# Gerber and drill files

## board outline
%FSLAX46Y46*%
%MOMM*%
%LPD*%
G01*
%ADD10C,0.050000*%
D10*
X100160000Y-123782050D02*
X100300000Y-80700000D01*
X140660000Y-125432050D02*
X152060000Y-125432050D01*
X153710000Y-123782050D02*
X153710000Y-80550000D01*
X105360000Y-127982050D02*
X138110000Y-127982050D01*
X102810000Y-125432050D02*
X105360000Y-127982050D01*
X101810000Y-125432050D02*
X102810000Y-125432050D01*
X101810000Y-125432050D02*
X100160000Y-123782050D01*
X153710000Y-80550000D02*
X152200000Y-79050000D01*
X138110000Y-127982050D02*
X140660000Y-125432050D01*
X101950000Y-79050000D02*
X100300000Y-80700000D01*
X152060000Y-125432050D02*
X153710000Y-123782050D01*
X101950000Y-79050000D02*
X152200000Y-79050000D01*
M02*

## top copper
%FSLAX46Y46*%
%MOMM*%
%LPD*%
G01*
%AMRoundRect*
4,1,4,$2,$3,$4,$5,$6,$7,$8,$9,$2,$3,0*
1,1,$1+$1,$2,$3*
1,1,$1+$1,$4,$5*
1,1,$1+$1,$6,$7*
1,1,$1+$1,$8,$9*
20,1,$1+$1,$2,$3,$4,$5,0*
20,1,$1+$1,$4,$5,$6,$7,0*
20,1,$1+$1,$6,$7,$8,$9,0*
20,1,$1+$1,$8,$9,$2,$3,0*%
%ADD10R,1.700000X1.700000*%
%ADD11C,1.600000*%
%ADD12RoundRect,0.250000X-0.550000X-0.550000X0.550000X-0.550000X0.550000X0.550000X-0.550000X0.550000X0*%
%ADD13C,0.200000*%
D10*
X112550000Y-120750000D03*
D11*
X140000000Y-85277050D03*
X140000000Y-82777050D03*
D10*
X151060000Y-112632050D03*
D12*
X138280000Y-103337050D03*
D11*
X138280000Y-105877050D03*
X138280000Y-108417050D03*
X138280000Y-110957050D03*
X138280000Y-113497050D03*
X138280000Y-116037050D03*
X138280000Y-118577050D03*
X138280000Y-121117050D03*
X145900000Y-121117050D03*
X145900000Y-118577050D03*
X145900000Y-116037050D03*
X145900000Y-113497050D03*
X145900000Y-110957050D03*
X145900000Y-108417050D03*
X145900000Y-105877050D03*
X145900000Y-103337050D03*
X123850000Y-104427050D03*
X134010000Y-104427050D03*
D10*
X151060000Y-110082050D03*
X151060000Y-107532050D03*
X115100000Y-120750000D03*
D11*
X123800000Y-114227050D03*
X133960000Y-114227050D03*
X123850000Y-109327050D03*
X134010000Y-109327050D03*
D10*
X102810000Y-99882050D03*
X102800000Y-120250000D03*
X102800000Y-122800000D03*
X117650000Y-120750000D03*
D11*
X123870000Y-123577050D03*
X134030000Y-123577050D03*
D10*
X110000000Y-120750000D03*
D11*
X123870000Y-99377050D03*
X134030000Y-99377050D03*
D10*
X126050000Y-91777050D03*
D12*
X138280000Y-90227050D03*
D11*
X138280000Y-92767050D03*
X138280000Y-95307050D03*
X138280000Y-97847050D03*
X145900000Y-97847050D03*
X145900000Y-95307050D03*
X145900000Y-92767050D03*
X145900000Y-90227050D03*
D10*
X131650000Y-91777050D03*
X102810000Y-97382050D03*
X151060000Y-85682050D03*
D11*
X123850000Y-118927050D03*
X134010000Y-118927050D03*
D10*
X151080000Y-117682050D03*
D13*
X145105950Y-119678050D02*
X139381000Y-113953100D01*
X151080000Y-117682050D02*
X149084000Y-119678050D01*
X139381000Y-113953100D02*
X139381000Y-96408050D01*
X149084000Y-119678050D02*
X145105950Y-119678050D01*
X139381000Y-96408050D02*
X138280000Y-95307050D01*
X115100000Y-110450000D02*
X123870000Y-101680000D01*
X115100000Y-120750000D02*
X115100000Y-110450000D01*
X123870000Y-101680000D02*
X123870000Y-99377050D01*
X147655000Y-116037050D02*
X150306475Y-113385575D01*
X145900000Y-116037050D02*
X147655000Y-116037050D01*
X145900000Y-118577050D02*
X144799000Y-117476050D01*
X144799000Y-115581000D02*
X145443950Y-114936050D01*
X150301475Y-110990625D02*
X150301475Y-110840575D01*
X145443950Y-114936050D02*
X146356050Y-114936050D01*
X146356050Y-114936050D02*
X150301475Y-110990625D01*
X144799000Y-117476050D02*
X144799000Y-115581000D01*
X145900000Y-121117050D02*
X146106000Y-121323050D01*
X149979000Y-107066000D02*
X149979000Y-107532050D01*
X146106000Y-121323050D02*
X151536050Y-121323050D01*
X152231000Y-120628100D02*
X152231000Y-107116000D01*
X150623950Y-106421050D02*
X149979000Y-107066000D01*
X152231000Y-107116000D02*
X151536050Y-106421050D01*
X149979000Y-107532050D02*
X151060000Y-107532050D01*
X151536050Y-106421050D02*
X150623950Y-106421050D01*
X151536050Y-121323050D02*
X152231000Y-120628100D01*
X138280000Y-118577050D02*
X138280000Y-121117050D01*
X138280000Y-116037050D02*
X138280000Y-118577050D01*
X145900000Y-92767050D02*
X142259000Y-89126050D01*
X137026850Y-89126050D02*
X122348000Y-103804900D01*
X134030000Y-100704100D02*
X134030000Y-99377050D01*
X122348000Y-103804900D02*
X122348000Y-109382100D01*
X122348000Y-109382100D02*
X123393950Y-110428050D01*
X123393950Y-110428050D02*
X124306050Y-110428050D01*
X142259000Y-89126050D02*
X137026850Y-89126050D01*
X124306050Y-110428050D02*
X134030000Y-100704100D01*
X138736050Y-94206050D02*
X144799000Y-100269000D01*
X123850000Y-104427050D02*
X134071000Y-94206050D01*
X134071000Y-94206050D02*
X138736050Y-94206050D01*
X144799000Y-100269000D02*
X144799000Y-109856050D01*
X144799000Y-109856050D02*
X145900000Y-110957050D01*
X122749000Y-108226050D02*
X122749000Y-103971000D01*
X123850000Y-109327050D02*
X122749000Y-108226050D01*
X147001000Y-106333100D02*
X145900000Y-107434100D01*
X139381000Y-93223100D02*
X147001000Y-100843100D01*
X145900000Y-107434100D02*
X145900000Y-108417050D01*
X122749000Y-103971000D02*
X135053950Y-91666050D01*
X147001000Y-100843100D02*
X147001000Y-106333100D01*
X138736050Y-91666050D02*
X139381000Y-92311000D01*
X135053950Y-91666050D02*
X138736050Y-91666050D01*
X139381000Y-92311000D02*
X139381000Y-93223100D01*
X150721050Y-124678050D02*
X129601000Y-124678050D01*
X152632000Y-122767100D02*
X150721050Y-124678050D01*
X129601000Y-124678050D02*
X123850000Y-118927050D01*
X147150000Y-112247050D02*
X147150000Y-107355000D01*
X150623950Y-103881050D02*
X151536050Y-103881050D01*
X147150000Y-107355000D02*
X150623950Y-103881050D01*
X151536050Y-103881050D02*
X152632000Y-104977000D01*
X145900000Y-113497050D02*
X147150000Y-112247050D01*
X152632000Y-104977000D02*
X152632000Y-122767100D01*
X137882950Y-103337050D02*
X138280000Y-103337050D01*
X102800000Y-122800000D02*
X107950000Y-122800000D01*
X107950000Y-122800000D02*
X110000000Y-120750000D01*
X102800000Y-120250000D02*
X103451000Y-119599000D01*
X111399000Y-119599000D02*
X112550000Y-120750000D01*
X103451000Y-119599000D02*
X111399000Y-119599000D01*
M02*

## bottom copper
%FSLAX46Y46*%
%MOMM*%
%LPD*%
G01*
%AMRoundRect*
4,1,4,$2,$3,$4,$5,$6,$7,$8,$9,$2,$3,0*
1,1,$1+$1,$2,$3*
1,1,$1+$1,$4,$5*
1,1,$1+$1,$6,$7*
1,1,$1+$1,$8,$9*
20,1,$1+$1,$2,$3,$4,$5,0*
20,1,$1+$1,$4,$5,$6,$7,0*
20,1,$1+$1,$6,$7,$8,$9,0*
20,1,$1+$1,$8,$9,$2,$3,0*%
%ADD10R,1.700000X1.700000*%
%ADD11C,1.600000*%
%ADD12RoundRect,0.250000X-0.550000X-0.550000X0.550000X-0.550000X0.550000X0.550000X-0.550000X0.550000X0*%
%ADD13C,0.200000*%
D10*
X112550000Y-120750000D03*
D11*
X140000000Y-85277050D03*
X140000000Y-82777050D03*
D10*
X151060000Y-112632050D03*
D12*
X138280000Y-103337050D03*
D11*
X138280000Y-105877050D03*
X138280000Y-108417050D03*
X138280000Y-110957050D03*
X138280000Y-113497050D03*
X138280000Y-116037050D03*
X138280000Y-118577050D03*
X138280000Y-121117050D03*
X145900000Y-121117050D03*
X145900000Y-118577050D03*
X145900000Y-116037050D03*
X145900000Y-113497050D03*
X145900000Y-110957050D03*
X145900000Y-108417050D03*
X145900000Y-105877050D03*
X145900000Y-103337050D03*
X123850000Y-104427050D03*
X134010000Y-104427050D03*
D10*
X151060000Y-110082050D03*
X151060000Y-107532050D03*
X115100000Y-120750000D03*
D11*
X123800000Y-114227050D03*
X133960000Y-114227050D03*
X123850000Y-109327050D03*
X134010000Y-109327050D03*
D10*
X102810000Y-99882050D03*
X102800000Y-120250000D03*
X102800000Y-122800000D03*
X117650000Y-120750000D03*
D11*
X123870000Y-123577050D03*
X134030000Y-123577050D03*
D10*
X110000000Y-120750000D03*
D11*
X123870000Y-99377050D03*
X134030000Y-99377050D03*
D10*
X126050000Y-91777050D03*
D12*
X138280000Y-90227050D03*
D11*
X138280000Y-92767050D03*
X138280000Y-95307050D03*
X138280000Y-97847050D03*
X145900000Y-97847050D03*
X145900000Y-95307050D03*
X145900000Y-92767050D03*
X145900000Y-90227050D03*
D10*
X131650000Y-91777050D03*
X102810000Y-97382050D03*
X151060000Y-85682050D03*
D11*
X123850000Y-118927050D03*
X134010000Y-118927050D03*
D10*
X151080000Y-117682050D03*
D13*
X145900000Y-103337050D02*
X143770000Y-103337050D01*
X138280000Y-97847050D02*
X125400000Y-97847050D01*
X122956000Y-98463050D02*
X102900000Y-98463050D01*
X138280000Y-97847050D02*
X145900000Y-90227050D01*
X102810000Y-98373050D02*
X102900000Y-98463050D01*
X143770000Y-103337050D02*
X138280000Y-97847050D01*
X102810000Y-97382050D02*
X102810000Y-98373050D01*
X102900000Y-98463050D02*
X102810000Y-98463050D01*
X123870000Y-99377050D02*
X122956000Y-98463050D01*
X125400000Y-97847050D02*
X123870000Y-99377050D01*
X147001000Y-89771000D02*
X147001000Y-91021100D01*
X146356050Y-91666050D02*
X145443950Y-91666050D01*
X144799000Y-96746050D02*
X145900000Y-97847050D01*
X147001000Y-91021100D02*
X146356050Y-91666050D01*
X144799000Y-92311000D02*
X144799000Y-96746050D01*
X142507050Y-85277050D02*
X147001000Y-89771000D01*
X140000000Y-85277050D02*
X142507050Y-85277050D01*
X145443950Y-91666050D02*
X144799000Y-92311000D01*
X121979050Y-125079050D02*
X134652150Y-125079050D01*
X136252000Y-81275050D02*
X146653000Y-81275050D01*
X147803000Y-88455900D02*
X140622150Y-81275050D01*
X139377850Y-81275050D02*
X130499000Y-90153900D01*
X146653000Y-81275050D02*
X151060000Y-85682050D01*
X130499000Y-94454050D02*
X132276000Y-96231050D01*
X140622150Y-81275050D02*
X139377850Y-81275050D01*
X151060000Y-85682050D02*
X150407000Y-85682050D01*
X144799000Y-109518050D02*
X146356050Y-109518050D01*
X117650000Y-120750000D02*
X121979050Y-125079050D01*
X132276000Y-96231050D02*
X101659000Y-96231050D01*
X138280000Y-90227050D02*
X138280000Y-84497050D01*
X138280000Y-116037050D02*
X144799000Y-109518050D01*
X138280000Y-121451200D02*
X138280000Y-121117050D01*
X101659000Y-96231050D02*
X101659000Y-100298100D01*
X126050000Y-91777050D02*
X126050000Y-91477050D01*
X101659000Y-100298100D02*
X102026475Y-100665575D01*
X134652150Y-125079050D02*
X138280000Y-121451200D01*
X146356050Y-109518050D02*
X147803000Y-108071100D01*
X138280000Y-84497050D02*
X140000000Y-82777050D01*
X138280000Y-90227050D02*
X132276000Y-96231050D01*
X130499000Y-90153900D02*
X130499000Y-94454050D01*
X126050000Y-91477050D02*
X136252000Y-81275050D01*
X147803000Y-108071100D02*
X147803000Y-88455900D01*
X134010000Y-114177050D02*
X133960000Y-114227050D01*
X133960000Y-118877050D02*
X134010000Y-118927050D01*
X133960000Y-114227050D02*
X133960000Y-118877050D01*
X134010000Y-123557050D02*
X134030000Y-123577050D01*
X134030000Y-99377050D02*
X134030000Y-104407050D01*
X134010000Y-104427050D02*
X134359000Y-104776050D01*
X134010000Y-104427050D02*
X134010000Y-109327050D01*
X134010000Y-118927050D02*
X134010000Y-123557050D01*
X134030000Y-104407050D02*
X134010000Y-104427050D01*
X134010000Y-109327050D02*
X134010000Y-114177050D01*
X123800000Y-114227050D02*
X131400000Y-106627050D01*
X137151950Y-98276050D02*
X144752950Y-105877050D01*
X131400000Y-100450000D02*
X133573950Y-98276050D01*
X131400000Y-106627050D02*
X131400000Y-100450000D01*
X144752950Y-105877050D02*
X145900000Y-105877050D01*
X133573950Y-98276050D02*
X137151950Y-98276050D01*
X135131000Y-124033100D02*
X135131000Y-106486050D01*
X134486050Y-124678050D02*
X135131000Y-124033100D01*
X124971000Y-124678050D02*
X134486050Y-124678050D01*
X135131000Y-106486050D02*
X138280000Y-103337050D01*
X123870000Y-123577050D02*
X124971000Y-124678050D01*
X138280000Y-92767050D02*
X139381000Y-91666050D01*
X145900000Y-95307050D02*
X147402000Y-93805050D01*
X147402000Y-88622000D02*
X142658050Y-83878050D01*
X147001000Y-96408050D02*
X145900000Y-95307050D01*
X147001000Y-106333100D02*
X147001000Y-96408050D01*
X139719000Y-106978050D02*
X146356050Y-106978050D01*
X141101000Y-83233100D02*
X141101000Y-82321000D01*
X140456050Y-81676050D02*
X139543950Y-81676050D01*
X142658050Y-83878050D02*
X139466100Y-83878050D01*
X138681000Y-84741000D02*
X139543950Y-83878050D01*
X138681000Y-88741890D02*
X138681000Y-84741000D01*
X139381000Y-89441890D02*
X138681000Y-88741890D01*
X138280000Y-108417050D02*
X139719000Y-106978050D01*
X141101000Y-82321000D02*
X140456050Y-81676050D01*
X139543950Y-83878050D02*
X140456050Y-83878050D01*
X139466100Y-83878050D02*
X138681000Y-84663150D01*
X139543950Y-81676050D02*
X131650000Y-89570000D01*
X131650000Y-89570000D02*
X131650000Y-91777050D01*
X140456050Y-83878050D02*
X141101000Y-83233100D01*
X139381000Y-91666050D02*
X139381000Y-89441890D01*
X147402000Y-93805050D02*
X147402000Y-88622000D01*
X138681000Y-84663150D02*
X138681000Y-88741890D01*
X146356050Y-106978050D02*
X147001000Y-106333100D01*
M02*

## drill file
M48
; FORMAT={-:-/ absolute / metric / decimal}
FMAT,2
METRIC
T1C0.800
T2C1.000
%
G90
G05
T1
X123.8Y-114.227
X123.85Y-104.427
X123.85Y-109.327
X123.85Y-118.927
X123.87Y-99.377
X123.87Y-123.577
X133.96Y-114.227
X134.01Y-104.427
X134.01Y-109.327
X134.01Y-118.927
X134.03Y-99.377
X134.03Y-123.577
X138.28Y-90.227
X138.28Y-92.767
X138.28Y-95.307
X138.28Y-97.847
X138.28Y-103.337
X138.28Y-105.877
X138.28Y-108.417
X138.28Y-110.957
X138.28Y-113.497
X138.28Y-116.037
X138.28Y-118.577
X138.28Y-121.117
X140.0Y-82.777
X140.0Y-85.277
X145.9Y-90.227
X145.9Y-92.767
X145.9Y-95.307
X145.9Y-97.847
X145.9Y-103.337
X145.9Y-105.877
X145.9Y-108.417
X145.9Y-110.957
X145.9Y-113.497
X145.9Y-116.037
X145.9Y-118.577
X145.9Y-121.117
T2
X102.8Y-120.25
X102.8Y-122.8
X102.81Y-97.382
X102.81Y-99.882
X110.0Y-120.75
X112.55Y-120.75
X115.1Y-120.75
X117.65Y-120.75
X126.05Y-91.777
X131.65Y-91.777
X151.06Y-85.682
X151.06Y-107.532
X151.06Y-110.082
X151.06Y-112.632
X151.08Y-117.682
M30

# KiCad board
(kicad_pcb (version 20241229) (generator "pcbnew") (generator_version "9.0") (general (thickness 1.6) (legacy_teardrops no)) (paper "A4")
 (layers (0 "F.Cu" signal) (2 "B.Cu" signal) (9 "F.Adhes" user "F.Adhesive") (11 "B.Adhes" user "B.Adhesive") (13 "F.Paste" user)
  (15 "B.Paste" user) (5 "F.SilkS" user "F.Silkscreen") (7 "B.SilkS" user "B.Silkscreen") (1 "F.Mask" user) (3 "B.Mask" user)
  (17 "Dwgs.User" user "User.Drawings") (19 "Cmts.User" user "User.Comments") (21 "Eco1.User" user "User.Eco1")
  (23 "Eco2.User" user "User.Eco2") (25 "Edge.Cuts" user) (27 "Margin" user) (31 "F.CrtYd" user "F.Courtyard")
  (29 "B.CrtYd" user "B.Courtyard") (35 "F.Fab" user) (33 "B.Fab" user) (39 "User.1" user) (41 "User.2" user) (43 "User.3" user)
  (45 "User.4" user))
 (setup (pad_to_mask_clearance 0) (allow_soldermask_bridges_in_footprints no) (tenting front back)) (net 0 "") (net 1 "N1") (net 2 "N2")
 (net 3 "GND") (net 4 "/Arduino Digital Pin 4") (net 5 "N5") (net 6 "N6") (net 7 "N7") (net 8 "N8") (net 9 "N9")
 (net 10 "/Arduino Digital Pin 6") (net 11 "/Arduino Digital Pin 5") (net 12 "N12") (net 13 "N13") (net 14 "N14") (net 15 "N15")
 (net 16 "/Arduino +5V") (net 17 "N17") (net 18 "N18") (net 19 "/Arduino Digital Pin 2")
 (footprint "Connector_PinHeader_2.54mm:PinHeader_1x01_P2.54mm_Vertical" (layer "F.Cu") (at 112.55 120.75)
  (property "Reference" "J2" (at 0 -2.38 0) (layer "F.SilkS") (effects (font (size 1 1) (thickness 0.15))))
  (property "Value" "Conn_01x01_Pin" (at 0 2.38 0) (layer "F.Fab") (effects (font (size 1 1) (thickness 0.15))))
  (pad "1" thru_hole rect (at 0 0) (size 1.7 1.7) (drill 1) (layers "*.Cu" "*.Mask") (remove_unused_layers no) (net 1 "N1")))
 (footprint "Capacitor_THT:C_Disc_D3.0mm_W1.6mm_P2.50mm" (layer "F.Cu") (at 140 85.27705 90)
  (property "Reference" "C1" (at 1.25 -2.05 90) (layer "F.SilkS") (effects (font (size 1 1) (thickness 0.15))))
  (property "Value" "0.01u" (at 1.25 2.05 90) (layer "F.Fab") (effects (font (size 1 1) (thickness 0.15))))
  (pad "1" thru_hole circle (at 0 0 90) (size 1.6 1.6) (drill 0.8) (layers "*.Cu" "*.Mask") (remove_unused_layers no) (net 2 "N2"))
  (pad "2" thru_hole circle (at 2.5 0 90) (size 1.6 1.6) (drill 0.8) (layers "*.Cu" "*.Mask") (remove_unused_layers no) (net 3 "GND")))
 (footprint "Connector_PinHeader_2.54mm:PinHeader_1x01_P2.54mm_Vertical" (layer "F.Cu") (at 151.06 112.63205)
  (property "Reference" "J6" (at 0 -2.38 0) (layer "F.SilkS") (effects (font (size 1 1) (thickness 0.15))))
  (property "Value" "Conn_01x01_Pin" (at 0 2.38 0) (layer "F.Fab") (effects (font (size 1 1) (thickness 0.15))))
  (pad "1" thru_hole rect (at 0 0) (size 1.7 1.7) (drill 1) (layers "*.Cu" "*.Mask") (remove_unused_layers no)
   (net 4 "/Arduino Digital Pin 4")))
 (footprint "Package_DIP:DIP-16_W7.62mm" (layer "F.Cu") (at 138.28 103.33705)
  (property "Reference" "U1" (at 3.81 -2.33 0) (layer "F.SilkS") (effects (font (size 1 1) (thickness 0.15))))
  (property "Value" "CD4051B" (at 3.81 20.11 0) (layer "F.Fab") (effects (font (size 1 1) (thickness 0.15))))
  (pad "1" thru_hole roundrect (at 0 0) (size 1.6 1.6) (drill 0.8) (layers "*.Cu" "*.Mask") (remove_unused_layers no)
   (roundrect_rratio 0.15625) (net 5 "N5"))
  (pad "2" thru_hole circle (at 0 2.54) (size 1.6 1.6) (drill 0.8) (layers "*.Cu" "*.Mask") (remove_unused_layers no) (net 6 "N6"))
  (pad "3" thru_hole circle (at 0 5.08) (size 1.6 1.6) (drill 0.8) (layers "*.Cu" "*.Mask") (remove_unused_layers no) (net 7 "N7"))
  (pad "4" thru_hole circle (at 0 7.62) (size 1.6 1.6) (drill 0.8) (layers "*.Cu" "*.Mask") (remove_unused_layers no) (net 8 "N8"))
  (pad "5" thru_hole circle (at 0 10.16) (size 1.6 1.6) (drill 0.8) (layers "*.Cu" "*.Mask") (remove_unused_layers no) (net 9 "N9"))
  (pad "6" thru_hole circle (at 0 12.7) (size 1.6 1.6) (drill 0.8) (layers "*.Cu" "*.Mask") (remove_unused_layers no) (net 3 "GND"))
  (pad "7" thru_hole circle (at 0 15.24) (size 1.6 1.6) (drill 0.8) (layers "*.Cu" "*.Mask") (remove_unused_layers no) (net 3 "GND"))
  (pad "8" thru_hole circle (at 0 17.78) (size 1.6 1.6) (drill 0.8) (layers "*.Cu" "*.Mask") (remove_unused_layers no) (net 3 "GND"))
  (pad "9" thru_hole circle (at 7.62 17.78) (size 1.6 1.6) (drill 0.8) (layers "*.Cu" "*.Mask") (remove_unused_layers no)
   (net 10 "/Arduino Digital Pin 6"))
  (pad "10" thru_hole circle (at 7.62 15.24) (size 1.6 1.6) (drill 0.8) (layers "*.Cu" "*.Mask") (remove_unused_layers no)
   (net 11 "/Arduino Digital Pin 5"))
  (pad "11" thru_hole circle (at 7.62 12.7) (size 1.6 1.6) (drill 0.8) (layers "*.Cu" "*.Mask") (remove_unused_layers no)
   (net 4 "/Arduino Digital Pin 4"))
  (pad "12" thru_hole circle (at 7.62 10.16) (size 1.6 1.6) (drill 0.8) (layers "*.Cu" "*.Mask") (remove_unused_layers no) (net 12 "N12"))
  (pad "13" thru_hole circle (at 7.62 7.62) (size 1.6 1.6) (drill 0.8) (layers "*.Cu" "*.Mask") (remove_unused_layers no) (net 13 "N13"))
  (pad "14" thru_hole circle (at 7.62 5.08) (size 1.6 1.6) (drill 0.8) (layers "*.Cu" "*.Mask") (remove_unused_layers no) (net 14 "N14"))
  (pad "15" thru_hole circle (at 7.62 2.54) (size 1.6 1.6) (drill 0.8) (layers "*.Cu" "*.Mask") (remove_unused_layers no) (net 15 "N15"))
  (pad "16" thru_hole circle (at 7.62 0) (size 1.6 1.6) (drill 0.8) (layers "*.Cu" "*.Mask") (remove_unused_layers no)
   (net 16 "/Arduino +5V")))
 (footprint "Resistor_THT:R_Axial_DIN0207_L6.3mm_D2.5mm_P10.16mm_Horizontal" (layer "F.Cu") (at 123.85 104.42705)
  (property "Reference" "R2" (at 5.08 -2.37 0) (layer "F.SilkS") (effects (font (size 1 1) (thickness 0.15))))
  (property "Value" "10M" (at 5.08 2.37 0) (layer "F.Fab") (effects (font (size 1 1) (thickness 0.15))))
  (pad "1" thru_hole circle (at 0 0) (size 1.6 1.6) (drill 0.8) (layers "*.Cu" "*.Mask") (remove_unused_layers no) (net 13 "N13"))
  (pad "2" thru_hole circle (at 10.16 0) (size 1.6 1.6) (drill 0.8) (layers "*.Cu" "*.Mask") (remove_unused_layers no) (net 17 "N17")))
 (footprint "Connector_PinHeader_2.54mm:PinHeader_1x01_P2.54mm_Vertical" (layer "F.Cu") (at 151.06 110.08205)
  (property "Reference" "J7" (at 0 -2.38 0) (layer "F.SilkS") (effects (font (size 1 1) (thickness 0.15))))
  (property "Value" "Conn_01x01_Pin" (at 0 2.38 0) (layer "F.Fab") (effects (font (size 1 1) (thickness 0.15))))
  (pad "1" thru_hole rect (at 0 0) (size 1.7 1.7) (drill 1) (layers "*.Cu" "*.Mask") (remove_unused_layers no)
   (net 11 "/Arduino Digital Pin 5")))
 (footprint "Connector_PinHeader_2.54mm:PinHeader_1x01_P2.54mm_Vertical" (layer "F.Cu") (at 151.06 107.53205)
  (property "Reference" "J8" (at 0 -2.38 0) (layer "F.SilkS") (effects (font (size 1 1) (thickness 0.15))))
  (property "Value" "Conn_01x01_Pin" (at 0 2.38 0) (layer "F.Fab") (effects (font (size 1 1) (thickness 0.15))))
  (pad "1" thru_hole rect (at 0 0) (size 1.7 1.7) (drill 1) (layers "*.Cu" "*.Mask") (remove_unused_layers no)
   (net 10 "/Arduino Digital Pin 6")))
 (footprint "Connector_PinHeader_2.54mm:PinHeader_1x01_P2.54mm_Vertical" (layer "F.Cu") (at 115.1 120.75)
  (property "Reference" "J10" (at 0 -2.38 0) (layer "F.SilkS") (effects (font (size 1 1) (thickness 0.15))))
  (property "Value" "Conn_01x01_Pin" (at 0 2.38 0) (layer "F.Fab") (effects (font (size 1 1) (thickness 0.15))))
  (pad "1" thru_hole rect (at 0 0) (size 1.7 1.7) (drill 1) (layers "*.Cu" "*.Mask") (remove_unused_layers no) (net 16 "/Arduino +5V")))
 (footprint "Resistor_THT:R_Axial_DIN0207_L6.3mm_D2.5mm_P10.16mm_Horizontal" (layer "F.Cu") (at 123.8 114.22705)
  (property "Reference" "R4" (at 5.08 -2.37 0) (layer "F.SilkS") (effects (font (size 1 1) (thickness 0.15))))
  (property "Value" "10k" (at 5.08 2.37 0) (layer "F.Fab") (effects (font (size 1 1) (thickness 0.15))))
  (pad "1" thru_hole circle (at 0 0) (size 1.6 1.6) (drill 0.8) (layers "*.Cu" "*.Mask") (remove_unused_layers no) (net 15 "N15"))
  (pad "2" thru_hole circle (at 10.16 0) (size 1.6 1.6) (drill 0.8) (layers "*.Cu" "*.Mask") (remove_unused_layers no) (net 17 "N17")))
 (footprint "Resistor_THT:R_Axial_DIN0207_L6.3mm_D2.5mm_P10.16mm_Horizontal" (layer "F.Cu") (at 123.85 109.32705)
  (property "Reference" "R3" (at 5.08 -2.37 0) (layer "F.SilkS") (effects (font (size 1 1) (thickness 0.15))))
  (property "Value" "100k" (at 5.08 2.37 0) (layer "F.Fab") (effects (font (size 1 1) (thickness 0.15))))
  (pad "1" thru_hole circle (at 0 0) (size 1.6 1.6) (drill 0.8) (layers "*.Cu" "*.Mask") (remove_unused_layers no) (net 14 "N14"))
  (pad "2" thru_hole circle (at 10.16 0) (size 1.6 1.6) (drill 0.8) (layers "*.Cu" "*.Mask") (remove_unused_layers no) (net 17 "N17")))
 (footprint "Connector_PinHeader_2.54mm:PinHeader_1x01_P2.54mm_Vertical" (layer "F.Cu") (at 102.81 99.88205)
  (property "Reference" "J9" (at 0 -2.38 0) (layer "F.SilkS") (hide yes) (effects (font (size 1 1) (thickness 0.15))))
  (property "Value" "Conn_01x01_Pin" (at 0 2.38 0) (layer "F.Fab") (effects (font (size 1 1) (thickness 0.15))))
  (pad "1" thru_hole rect (at 0 0) (size 1.7 1.7) (drill 1) (layers "*.Cu" "*.Mask") (remove_unused_layers no) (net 3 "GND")))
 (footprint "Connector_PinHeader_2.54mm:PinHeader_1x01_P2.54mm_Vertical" (layer "F.Cu") (at 102.8 120.25)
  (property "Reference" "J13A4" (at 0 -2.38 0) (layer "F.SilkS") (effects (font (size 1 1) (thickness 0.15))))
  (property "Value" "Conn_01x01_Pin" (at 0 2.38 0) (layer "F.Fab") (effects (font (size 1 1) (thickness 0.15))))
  (pad "1" thru_hole rect (at 0 0) (size 1.7 1.7) (drill 1) (layers "*.Cu" "*.Mask") (remove_unused_layers no) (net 1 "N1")))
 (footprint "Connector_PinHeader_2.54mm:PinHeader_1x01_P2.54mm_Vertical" (layer "F.Cu") (at 102.8 122.8)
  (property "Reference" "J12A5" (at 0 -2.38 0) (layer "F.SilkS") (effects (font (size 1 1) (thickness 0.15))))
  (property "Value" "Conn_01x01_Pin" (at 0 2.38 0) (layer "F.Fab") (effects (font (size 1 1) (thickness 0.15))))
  (pad "1" thru_hole rect (at 0 0) (size 1.7 1.7) (drill 1) (layers "*.Cu" "*.Mask") (remove_unused_layers no) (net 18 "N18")))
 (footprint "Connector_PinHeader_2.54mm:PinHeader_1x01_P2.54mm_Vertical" (layer "F.Cu") (at 117.65 120.75)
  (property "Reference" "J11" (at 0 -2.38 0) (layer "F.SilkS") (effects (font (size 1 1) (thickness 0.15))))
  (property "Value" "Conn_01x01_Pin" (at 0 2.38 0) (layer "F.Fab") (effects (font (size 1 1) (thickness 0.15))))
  (pad "1" thru_hole rect (at 0 0) (size 1.7 1.7) (drill 1) (layers "*.Cu" "*.Mask") (remove_unused_layers no) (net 3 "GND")))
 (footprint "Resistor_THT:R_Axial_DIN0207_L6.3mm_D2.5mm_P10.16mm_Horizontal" (layer "F.Cu") (at 123.87 123.57705)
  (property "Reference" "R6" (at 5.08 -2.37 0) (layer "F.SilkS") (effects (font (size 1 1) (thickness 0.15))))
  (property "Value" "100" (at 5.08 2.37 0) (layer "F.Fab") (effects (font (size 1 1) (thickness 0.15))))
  (pad "1" thru_hole circle (at 0 0) (size 1.6 1.6) (drill 0.8) (layers "*.Cu" "*.Mask") (remove_unused_layers no) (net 5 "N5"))
  (pad "2" thru_hole circle (at 10.16 0) (size 1.6 1.6) (drill 0.8) (layers "*.Cu" "*.Mask") (remove_unused_layers no) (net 17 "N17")))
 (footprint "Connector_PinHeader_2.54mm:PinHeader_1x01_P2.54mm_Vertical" (layer "F.Cu") (at 110 120.75)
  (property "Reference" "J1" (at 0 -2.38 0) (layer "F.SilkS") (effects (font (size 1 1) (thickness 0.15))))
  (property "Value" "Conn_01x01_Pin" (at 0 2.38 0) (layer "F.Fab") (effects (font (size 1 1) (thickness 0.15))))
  (pad "1" thru_hole rect (at 0 0) (size 1.7 1.7) (drill 1) (layers "*.Cu" "*.Mask") (remove_unused_layers no) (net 18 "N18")))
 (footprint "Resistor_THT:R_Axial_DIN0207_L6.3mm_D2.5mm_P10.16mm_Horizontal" (layer "F.Cu") (at 123.87 99.37705)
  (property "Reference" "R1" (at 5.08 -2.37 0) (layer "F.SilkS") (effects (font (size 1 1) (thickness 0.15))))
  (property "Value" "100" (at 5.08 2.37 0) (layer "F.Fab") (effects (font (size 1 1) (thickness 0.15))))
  (pad "1" thru_hole circle (at 0 0) (size 1.6 1.6) (drill 0.8) (layers "*.Cu" "*.Mask") (remove_unused_layers no) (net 16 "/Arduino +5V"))
  (pad "2" thru_hole circle (at 10.16 0) (size 1.6 1.6) (drill 0.8) (layers "*.Cu" "*.Mask") (remove_unused_layers no) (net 17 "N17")))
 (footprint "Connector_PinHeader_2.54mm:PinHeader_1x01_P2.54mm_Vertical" (layer "F.Cu") (at 126.05 91.77705)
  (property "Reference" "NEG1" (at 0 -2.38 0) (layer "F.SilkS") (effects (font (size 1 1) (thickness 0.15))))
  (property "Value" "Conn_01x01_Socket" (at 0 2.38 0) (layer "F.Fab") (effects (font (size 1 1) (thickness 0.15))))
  (pad "1" thru_hole rect (at 0 0) (size 1.7 1.7) (drill 1) (layers "*.Cu" "*.Mask") (remove_unused_layers no) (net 3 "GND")))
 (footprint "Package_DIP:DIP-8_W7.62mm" (layer "F.Cu") (at 138.28 90.22705)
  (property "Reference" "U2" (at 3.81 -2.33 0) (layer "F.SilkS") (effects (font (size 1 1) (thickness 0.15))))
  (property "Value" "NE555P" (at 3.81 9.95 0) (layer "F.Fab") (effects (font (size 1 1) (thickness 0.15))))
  (pad "1" thru_hole roundrect (at 0 0) (size 1.6 1.6) (drill 0.8) (layers "*.Cu" "*.Mask") (remove_unused_layers no)
   (roundrect_rratio 0.15625) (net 3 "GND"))
  (pad "2" thru_hole circle (at 0 2.54) (size 1.6 1.6) (drill 0.8) (layers "*.Cu" "*.Mask") (remove_unused_layers no) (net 7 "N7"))
  (pad "3" thru_hole circle (at 0 5.08) (size 1.6 1.6) (drill 0.8) (layers "*.Cu" "*.Mask") (remove_unused_layers no)
   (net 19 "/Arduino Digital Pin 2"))
  (pad "4" thru_hole circle (at 0 7.62) (size 1.6 1.6) (drill 0.8) (layers "*.Cu" "*.Mask") (remove_unused_layers no)
   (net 16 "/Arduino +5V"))
  (pad "5" thru_hole circle (at 7.62 7.62) (size 1.6 1.6) (drill 0.8) (layers "*.Cu" "*.Mask") (remove_unused_layers no) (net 2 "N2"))
  (pad "6" thru_hole circle (at 7.62 5.08) (size 1.6 1.6) (drill 0.8) (layers "*.Cu" "*.Mask") (remove_unused_layers no) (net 7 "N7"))
  (pad "7" thru_hole circle (at 7.62 2.54) (size 1.6 1.6) (drill 0.8) (layers "*.Cu" "*.Mask") (remove_unused_layers no) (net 17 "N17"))
  (pad "8" thru_hole circle (at 7.62 0) (size 1.6 1.6) (drill 0.8) (layers "*.Cu" "*.Mask") (remove_unused_layers no)
   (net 16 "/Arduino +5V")))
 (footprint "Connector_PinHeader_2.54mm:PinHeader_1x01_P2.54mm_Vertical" (layer "F.Cu") (at 131.65 91.77705)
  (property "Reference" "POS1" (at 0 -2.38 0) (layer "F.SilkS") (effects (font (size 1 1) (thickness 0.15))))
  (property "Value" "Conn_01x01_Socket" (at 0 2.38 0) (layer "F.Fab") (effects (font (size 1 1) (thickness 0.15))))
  (pad "1" thru_hole rect (at 0 0) (size 1.7 1.7) (drill 1) (layers "*.Cu" "*.Mask") (remove_unused_layers no) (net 7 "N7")))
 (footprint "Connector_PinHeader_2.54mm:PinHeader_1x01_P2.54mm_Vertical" (layer "F.Cu") (at 102.81 97.38205)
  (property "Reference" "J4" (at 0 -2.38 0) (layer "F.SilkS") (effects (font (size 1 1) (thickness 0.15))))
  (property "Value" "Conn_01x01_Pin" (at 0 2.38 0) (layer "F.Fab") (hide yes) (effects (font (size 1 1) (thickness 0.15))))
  (pad "1" thru_hole rect (at 0 0) (size 1.7 1.7) (drill 1) (layers "*.Cu" "*.Mask") (remove_unused_layers no) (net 16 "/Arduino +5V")))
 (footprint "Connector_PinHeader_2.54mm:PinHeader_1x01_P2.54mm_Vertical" (layer "F.Cu") (at 151.06 85.68205)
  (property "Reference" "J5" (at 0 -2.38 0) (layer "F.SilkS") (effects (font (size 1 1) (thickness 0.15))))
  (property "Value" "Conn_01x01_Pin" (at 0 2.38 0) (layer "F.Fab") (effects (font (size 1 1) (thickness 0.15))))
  (pad "1" thru_hole rect (at 0 0) (size 1.7 1.7) (drill 1) (layers "*.Cu" "*.Mask") (remove_unused_layers no) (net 3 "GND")))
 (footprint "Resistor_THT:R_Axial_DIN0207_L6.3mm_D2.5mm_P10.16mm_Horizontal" (layer "F.Cu") (at 123.85 118.92705)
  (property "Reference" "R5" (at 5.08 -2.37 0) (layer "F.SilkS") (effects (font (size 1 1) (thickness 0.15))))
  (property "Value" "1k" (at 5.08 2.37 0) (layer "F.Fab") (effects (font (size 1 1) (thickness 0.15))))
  (pad "1" thru_hole circle (at 0 0) (size 1.6 1.6) (drill 0.8) (layers "*.Cu" "*.Mask") (remove_unused_layers no) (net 12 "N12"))
  (pad "2" thru_hole circle (at 10.16 0) (size 1.6 1.6) (drill 0.8) (layers "*.Cu" "*.Mask") (remove_unused_layers no) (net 17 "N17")))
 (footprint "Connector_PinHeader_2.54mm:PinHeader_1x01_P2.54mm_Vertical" (layer "F.Cu") (at 151.08 117.68205)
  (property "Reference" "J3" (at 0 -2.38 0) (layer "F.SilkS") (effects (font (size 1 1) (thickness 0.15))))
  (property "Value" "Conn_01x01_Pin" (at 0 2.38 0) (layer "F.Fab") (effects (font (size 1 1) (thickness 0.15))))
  (pad "1" thru_hole rect (at 0 0) (size 1.7 1.7) (drill 1) (layers "*.Cu" "*.Mask") (remove_unused_layers no)
   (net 19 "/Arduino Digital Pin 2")))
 (gr_line (start 100.16 123.78205) (end 100.3 80.7) (stroke (width 0.05) (type default)) (layer "Edge.Cuts"))
 (gr_line (start 140.66 125.43205) (end 152.06 125.43205) (stroke (width 0.05) (type default)) (layer "Edge.Cuts"))
 (gr_line (start 153.71 123.78205) (end 153.71 80.55) (stroke (width 0.05) (type default)) (layer "Edge.Cuts"))
 (gr_line (start 105.36 127.98205) (end 138.11 127.98205) (stroke (width 0.05) (type default)) (layer "Edge.Cuts"))
 (gr_line (start 102.81 125.43205) (end 105.36 127.98205) (stroke (width 0.05) (type default)) (layer "Edge.Cuts"))
 (gr_line (start 101.81 125.43205) (end 102.81 125.43205) (stroke (width 0.05) (type default)) (layer "Edge.Cuts"))
 (gr_line (start 101.81 125.43205) (end 100.16 123.78205) (stroke (width 0.05) (type default)) (layer "Edge.Cuts"))
 (gr_line (start 153.71 80.55) (end 152.2 79.05) (stroke (width 0.05) (type default)) (layer "Edge.Cuts"))
 (gr_line (start 138.11 127.98205) (end 140.66 125.43205) (stroke (width 0.05) (type default)) (layer "Edge.Cuts"))
 (gr_line (start 101.95 79.05) (end 100.3 80.7) (stroke (width 0.05) (type default)) (layer "Edge.Cuts"))
 (gr_line (start 152.06 125.43205) (end 153.71 123.78205) (stroke (width 0.05) (type default)) (layer "Edge.Cuts"))
 (gr_line (start 101.95 79.05) (end 152.2 79.05) (stroke (width 0.05) (type default)) (layer "Edge.Cuts"))
 (segment (start 145.10595 119.67805) (end 139.381 113.9531) (width 0.2) (layer "F.Cu") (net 19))
 (segment (start 151.08 117.68205) (end 149.084 119.67805) (width 0.2) (layer "F.Cu") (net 19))
 (segment (start 139.381 113.9531) (end 139.381 96.40805) (width 0.2) (layer "F.Cu") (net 19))
 (segment (start 149.084 119.67805) (end 145.10595 119.67805) (width 0.2) (layer "F.Cu") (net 19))
 (segment (start 139.381 96.40805) (end 138.28 95.30705) (width 0.2) (layer "F.Cu") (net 19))
 (segment (start 115.1 110.45) (end 123.87 101.68) (width 0.2) (layer "F.Cu") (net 16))
 (segment (start 115.1 120.75) (end 115.1 110.45) (width 0.2) (layer "F.Cu") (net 16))
 (segment (start 123.87 101.68) (end 123.87 99.37705) (width 0.2) (layer "F.Cu") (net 16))
 (segment (start 145.9 103.33705) (end 143.77 103.33705) (width 0.2) (layer "B.Cu") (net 16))
 (segment (start 138.28 97.84705) (end 125.4 97.84705) (width 0.2) (layer "B.Cu") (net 16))
 (segment (start 122.956 98.46305) (end 102.9 98.46305) (width 0.2) (layer "B.Cu") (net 16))
 (segment (start 138.28 97.84705) (end 145.9 90.22705) (width 0.2) (layer "B.Cu") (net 16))
 (segment (start 102.81 98.37305) (end 102.9 98.46305) (width 0.2) (layer "B.Cu") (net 16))
 (segment (start 143.77 103.33705) (end 138.28 97.84705) (width 0.2) (layer "B.Cu") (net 16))
 (segment (start 102.81 97.38205) (end 102.81 98.37305) (width 0.2) (layer "B.Cu") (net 16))
 (segment (start 102.9 98.46305) (end 102.81 98.46305) (width 0.2) (layer "B.Cu") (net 16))
 (segment (start 123.87 99.37705) (end 122.956 98.46305) (width 0.2) (layer "B.Cu") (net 16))
 (segment (start 125.4 97.84705) (end 123.87 99.37705) (width 0.2) (layer "B.Cu") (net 16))
 (segment (start 147.655 116.03705) (end 150.306475 113.385575) (width 0.2) (layer "F.Cu") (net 4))
 (segment (start 145.9 116.03705) (end 147.655 116.03705) (width 0.2) (layer "F.Cu") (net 4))
 (segment (start 145.9 118.57705) (end 144.799 117.47605) (width 0.2) (layer "F.Cu") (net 11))
 (segment (start 144.799 115.581) (end 145.44395 114.93605) (width 0.2) (layer "F.Cu") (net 11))
 (segment (start 150.301475 110.990625) (end 150.301475 110.840575) (width 0.2) (layer "F.Cu") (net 11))
 (segment (start 145.44395 114.93605) (end 146.35605 114.93605) (width 0.2) (layer "F.Cu") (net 11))
 (segment (start 146.35605 114.93605) (end 150.301475 110.990625) (width 0.2) (layer "F.Cu") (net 11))
 (segment (start 144.799 117.47605) (end 144.799 115.581) (width 0.2) (layer "F.Cu") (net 11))
 (segment (start 145.9 121.11705) (end 146.106 121.32305) (width 0.2) (layer "F.Cu") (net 10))
 (segment (start 149.979 107.066) (end 149.979 107.53205) (width 0.2) (layer "F.Cu") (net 10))
 (segment (start 146.106 121.32305) (end 151.53605 121.32305) (width 0.2) (layer "F.Cu") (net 10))
 (segment (start 152.231 120.6281) (end 152.231 107.116) (width 0.2) (layer "F.Cu") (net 10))
 (segment (start 150.62395 106.42105) (end 149.979 107.066) (width 0.2) (layer "F.Cu") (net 10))
 (segment (start 152.231 107.116) (end 151.53605 106.42105) (width 0.2) (layer "F.Cu") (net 10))
 (segment (start 149.979 107.53205) (end 151.06 107.53205) (width 0.2) (layer "F.Cu") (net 10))
 (segment (start 151.53605 106.42105) (end 150.62395 106.42105) (width 0.2) (layer "F.Cu") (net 10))
 (segment (start 151.53605 121.32305) (end 152.231 120.6281) (width 0.2) (layer "F.Cu") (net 10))
 (segment (start 147.001 89.771) (end 147.001 91.0211) (width 0.2) (layer "B.Cu") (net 2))
 (segment (start 146.35605 91.66605) (end 145.44395 91.66605) (width 0.2) (layer "B.Cu") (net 2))
 (segment (start 144.799 96.74605) (end 145.9 97.84705) (width 0.2) (layer "B.Cu") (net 2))
 (segment (start 147.001 91.0211) (end 146.35605 91.66605) (width 0.2) (layer "B.Cu") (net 2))
 (segment (start 144.799 92.311) (end 144.799 96.74605) (width 0.2) (layer "B.Cu") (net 2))
 (segment (start 142.50705 85.27705) (end 147.001 89.771) (width 0.2) (layer "B.Cu") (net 2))
 (segment (start 140 85.27705) (end 142.50705 85.27705) (width 0.2) (layer "B.Cu") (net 2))
 (segment (start 145.44395 91.66605) (end 144.799 92.311) (width 0.2) (layer "B.Cu") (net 2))
 (segment (start 138.28 118.57705) (end 138.28 121.11705) (width 0.2) (layer "F.Cu") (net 3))
 (segment (start 138.28 116.03705) (end 138.28 118.57705) (width 0.2) (layer "F.Cu") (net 3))
 (segment (start 121.97905 125.07905) (end 134.65215 125.07905) (width 0.2) (layer "B.Cu") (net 3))
 (segment (start 136.252 81.27505) (end 146.653 81.27505) (width 0.2) (layer "B.Cu") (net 3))
 (segment (start 147.803 88.4559) (end 140.62215 81.27505) (width 0.2) (layer "B.Cu") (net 3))
 (segment (start 139.37785 81.27505) (end 130.499 90.1539) (width 0.2) (layer "B.Cu") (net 3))
 (segment (start 146.653 81.27505) (end 151.06 85.68205) (width 0.2) (layer "B.Cu") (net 3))
 (segment (start 130.499 94.45405) (end 132.276 96.23105) (width 0.2) (layer "B.Cu") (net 3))
 (segment (start 140.62215 81.27505) (end 139.37785 81.27505) (width 0.2) (layer "B.Cu") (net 3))
 (segment (start 151.06 85.68205) (end 150.407 85.68205) (width 0.2) (layer "B.Cu") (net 3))
 (segment (start 144.799 109.51805) (end 146.35605 109.51805) (width 0.2) (layer "B.Cu") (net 3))
 (segment (start 117.65 120.75) (end 121.97905 125.07905) (width 0.2) (layer "B.Cu") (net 3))
 (segment (start 132.276 96.23105) (end 101.659 96.23105) (width 0.2) (layer "B.Cu") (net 3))
 (segment (start 138.28 90.22705) (end 138.28 84.49705) (width 0.2) (layer "B.Cu") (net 3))
 (segment (start 138.28 116.03705) (end 144.799 109.51805) (width 0.2) (layer "B.Cu") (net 3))
 (segment (start 138.28 121.4512) (end 138.28 121.11705) (width 0.2) (layer "B.Cu") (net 3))
 (segment (start 101.659 96.23105) (end 101.659 100.2981) (width 0.2) (layer "B.Cu") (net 3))
 (segment (start 126.05 91.77705) (end 126.05 91.47705) (width 0.2) (layer "B.Cu") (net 3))
 (segment (start 101.659 100.2981) (end 102.026475 100.665575) (width 0.2) (layer "B.Cu") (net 3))
 (segment (start 134.65215 125.07905) (end 138.28 121.4512) (width 0.2) (layer "B.Cu") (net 3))
 (segment (start 146.35605 109.51805) (end 147.803 108.0711) (width 0.2) (layer "B.Cu") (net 3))
 (segment (start 138.28 84.49705) (end 140 82.77705) (width 0.2) (layer "B.Cu") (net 3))
 (segment (start 138.28 90.22705) (end 132.276 96.23105) (width 0.2) (layer "B.Cu") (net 3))
 (segment (start 130.499 90.1539) (end 130.499 94.45405) (width 0.2) (layer "B.Cu") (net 3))
 (segment (start 126.05 91.47705) (end 136.252 81.27505) (width 0.2) (layer "B.Cu") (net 3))
 (segment (start 147.803 108.0711) (end 147.803 88.4559) (width 0.2) (layer "B.Cu") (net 3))
 (segment (start 145.9 92.76705) (end 142.259 89.12605) (width 0.2) (layer "F.Cu") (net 17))
 (segment (start 137.02685 89.12605) (end 122.348 103.8049) (width 0.2) (layer "F.Cu") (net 17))
 (segment (start 134.03 100.7041) (end 134.03 99.37705) (width 0.2) (layer "F.Cu") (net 17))
 (segment (start 122.348 103.8049) (end 122.348 109.3821) (width 0.2) (layer "F.Cu") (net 17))
 (segment (start 122.348 109.3821) (end 123.39395 110.42805) (width 0.2) (layer "F.Cu") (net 17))
 (segment (start 123.39395 110.42805) (end 124.30605 110.42805) (width 0.2) (layer "F.Cu") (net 17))
 (segment (start 142.259 89.12605) (end 137.02685 89.12605) (width 0.2) (layer "F.Cu") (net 17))
 (segment (start 124.30605 110.42805) (end 134.03 100.7041) (width 0.2) (layer "F.Cu") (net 17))
 (segment (start 134.01 114.17705) (end 133.96 114.22705) (width 0.2) (layer "B.Cu") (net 17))
 (segment (start 133.96 118.87705) (end 134.01 118.92705) (width 0.2) (layer "B.Cu") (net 17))
 (segment (start 133.96 114.22705) (end 133.96 118.87705) (width 0.2) (layer "B.Cu") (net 17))
 (segment (start 134.01 123.55705) (end 134.03 123.57705) (width 0.2) (layer "B.Cu") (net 17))
 (segment (start 134.03 99.37705) (end 134.03 104.40705) (width 0.2) (layer "B.Cu") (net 17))
 (segment (start 134.01 104.42705) (end 134.359 104.77605) (width 0.2) (layer "B.Cu") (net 17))
 (segment (start 134.01 104.42705) (end 134.01 109.32705) (width 0.2) (layer "B.Cu") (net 17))
 (segment (start 134.01 118.92705) (end 134.01 123.55705) (width 0.2) (layer "B.Cu") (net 17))
 (segment (start 134.03 104.40705) (end 134.01 104.42705) (width 0.2) (layer "B.Cu") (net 17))
 (segment (start 134.01 109.32705) (end 134.01 114.17705) (width 0.2) (layer "B.Cu") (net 17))
 (segment (start 138.73605 94.20605) (end 144.799 100.269) (width 0.2) (layer "F.Cu") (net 13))
 (segment (start 123.85 104.42705) (end 134.071 94.20605) (width 0.2) (layer "F.Cu") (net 13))
 (segment (start 134.071 94.20605) (end 138.73605 94.20605) (width 0.2) (layer "F.Cu") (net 13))
 (segment (start 144.799 100.269) (end 144.799 109.85605) (width 0.2) (layer "F.Cu") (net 13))
 (segment (start 144.799 109.85605) (end 145.9 110.95705) (width 0.2) (layer "F.Cu") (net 13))
 (segment (start 122.749 108.22605) (end 122.749 103.971) (width 0.2) (layer "F.Cu") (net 14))
 (segment (start 123.85 109.32705) (end 122.749 108.22605) (width 0.2) (layer "F.Cu") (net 14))
 (segment (start 147.001 106.3331) (end 145.9 107.4341) (width 0.2) (layer "F.Cu") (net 14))
 (segment (start 139.381 93.2231) (end 147.001 100.8431) (width 0.2) (layer "F.Cu") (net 14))
 (segment (start 145.9 107.4341) (end 145.9 108.41705) (width 0.2) (layer "F.Cu") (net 14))
 (segment (start 122.749 103.971) (end 135.05395 91.66605) (width 0.2) (layer "F.Cu") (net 14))
 (segment (start 147.001 100.8431) (end 147.001 106.3331) (width 0.2) (layer "F.Cu") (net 14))
 (segment (start 138.73605 91.66605) (end 139.381 92.311) (width 0.2) (layer "F.Cu") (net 14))
 (segment (start 135.05395 91.66605) (end 138.73605 91.66605) (width 0.2) (layer "F.Cu") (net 14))
 (segment (start 139.381 92.311) (end 139.381 93.2231) (width 0.2) (layer "F.Cu") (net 14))
 (segment (start 123.8 114.22705) (end 131.4 106.62705) (width 0.2) (layer "B.Cu") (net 15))
 (segment (start 137.15195 98.27605) (end 144.75295 105.87705) (width 0.2) (layer "B.Cu") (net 15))
 (segment (start 131.4 100.45) (end 133.57395 98.27605) (width 0.2) (layer "B.Cu") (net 15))
 (segment (start 131.4 106.62705) (end 131.4 100.45) (width 0.2) (layer "B.Cu") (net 15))
 (segment (start 144.75295 105.87705) (end 145.9 105.87705) (width 0.2) (layer "B.Cu") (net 15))
 (segment (start 133.57395 98.27605) (end 137.15195 98.27605) (width 0.2) (layer "B.Cu") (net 15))
 (segment (start 150.72105 124.67805) (end 129.601 124.67805) (width 0.2) (layer "F.Cu") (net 12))
 (segment (start 152.632 122.7671) (end 150.72105 124.67805) (width 0.2) (layer "F.Cu") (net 12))
 (segment (start 129.601 124.67805) (end 123.85 118.92705) (width 0.2) (layer "F.Cu") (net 12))
 (segment (start 147.15 112.24705) (end 147.15 107.355) (width 0.2) (layer "F.Cu") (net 12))
 (segment (start 150.62395 103.88105) (end 151.53605 103.88105) (width 0.2) (layer "F.Cu") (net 12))
 (segment (start 147.15 107.355) (end 150.62395 103.88105) (width 0.2) (layer "F.Cu") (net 12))
 (segment (start 151.53605 103.88105) (end 152.632 104.977) (width 0.2) (layer "F.Cu") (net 12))
 (segment (start 145.9 113.49705) (end 147.15 112.24705) (width 0.2) (layer "F.Cu") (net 12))
 (segment (start 152.632 104.977) (end 152.632 122.7671) (width 0.2) (layer "F.Cu") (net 12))
 (segment (start 137.88295 103.33705) (end 138.28 103.33705) (width 0.2) (layer "F.Cu") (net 5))
 (segment (start 135.131 124.0331) (end 135.131 106.48605) (width 0.2) (layer "B.Cu") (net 5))
 (segment (start 134.48605 124.67805) (end 135.131 124.0331) (width 0.2) (layer "B.Cu") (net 5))
 (segment (start 124.971 124.67805) (end 134.48605 124.67805) (width 0.2) (layer "B.Cu") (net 5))
 (segment (start 135.131 106.48605) (end 138.28 103.33705) (width 0.2) (layer "B.Cu") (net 5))
 (segment (start 123.87 123.57705) (end 124.971 124.67805) (width 0.2) (layer "B.Cu") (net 5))
 (segment (start 138.28 92.76705) (end 139.381 91.66605) (width 0.2) (layer "B.Cu") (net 7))
 (segment (start 145.9 95.30705) (end 147.402 93.80505) (width 0.2) (layer "B.Cu") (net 7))
 (segment (start 147.402 88.622) (end 142.65805 83.87805) (width 0.2) (layer "B.Cu") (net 7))
 (segment (start 147.001 96.40805) (end 145.9 95.30705) (width 0.2) (layer "B.Cu") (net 7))
 (segment (start 147.001 106.3331) (end 147.001 96.40805) (width 0.2) (layer "B.Cu") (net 7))
 (segment (start 139.719 106.97805) (end 146.35605 106.97805) (width 0.2) (layer "B.Cu") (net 7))
 (segment (start 141.101 83.2331) (end 141.101 82.321) (width 0.2) (layer "B.Cu") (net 7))
 (segment (start 140.45605 81.67605) (end 139.54395 81.67605) (width 0.2) (layer "B.Cu") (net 7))
 (segment (start 142.65805 83.87805) (end 139.4661 83.87805) (width 0.2) (layer "B.Cu") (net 7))
 (segment (start 138.681 84.741) (end 139.54395 83.87805) (width 0.2) (layer "B.Cu") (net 7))
 (segment (start 138.681 88.74189) (end 138.681 84.741) (width 0.2) (layer "B.Cu") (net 7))
 (segment (start 139.381 89.44189) (end 138.681 88.74189) (width 0.2) (layer "B.Cu") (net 7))
 (segment (start 138.28 108.41705) (end 139.719 106.97805) (width 0.2) (layer "B.Cu") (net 7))
 (segment (start 141.101 82.321) (end 140.45605 81.67605) (width 0.2) (layer "B.Cu") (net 7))
 (segment (start 139.54395 83.87805) (end 140.45605 83.87805) (width 0.2) (layer "B.Cu") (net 7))
 (segment (start 139.4661 83.87805) (end 138.681 84.66315) (width 0.2) (layer "B.Cu") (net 7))
 (segment (start 139.54395 81.67605) (end 131.65 89.57) (width 0.2) (layer "B.Cu") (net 7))
 (segment (start 131.65 89.57) (end 131.65 91.77705) (width 0.2) (layer "B.Cu") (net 7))
 (segment (start 140.45605 83.87805) (end 141.101 83.2331) (width 0.2) (layer "B.Cu") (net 7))
 (segment (start 139.381 91.66605) (end 139.381 89.44189) (width 0.2) (layer "B.Cu") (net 7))
 (segment (start 147.402 93.80505) (end 147.402 88.622) (width 0.2) (layer "B.Cu") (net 7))
 (segment (start 138.681 84.66315) (end 138.681 88.74189) (width 0.2) (layer "B.Cu") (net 7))
 (segment (start 146.35605 106.97805) (end 147.001 106.3331) (width 0.2) (layer "B.Cu") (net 7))
 (segment (start 102.8 122.8) (end 107.95 122.8) (width 0.2) (layer "F.Cu") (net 18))
 (segment (start 107.95 122.8) (end 110 120.75) (width 0.2) (layer "F.Cu") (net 18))
 (segment (start 102.8 120.25) (end 103.451 119.599) (width 0.2) (layer "F.Cu") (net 1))
 (segment (start 111.399 119.599) (end 112.55 120.75) (width 0.2) (layer "F.Cu") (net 1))
 (segment (start 103.451 119.599) (end 111.399 119.599) (width 0.2) (layer "F.Cu") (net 1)))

